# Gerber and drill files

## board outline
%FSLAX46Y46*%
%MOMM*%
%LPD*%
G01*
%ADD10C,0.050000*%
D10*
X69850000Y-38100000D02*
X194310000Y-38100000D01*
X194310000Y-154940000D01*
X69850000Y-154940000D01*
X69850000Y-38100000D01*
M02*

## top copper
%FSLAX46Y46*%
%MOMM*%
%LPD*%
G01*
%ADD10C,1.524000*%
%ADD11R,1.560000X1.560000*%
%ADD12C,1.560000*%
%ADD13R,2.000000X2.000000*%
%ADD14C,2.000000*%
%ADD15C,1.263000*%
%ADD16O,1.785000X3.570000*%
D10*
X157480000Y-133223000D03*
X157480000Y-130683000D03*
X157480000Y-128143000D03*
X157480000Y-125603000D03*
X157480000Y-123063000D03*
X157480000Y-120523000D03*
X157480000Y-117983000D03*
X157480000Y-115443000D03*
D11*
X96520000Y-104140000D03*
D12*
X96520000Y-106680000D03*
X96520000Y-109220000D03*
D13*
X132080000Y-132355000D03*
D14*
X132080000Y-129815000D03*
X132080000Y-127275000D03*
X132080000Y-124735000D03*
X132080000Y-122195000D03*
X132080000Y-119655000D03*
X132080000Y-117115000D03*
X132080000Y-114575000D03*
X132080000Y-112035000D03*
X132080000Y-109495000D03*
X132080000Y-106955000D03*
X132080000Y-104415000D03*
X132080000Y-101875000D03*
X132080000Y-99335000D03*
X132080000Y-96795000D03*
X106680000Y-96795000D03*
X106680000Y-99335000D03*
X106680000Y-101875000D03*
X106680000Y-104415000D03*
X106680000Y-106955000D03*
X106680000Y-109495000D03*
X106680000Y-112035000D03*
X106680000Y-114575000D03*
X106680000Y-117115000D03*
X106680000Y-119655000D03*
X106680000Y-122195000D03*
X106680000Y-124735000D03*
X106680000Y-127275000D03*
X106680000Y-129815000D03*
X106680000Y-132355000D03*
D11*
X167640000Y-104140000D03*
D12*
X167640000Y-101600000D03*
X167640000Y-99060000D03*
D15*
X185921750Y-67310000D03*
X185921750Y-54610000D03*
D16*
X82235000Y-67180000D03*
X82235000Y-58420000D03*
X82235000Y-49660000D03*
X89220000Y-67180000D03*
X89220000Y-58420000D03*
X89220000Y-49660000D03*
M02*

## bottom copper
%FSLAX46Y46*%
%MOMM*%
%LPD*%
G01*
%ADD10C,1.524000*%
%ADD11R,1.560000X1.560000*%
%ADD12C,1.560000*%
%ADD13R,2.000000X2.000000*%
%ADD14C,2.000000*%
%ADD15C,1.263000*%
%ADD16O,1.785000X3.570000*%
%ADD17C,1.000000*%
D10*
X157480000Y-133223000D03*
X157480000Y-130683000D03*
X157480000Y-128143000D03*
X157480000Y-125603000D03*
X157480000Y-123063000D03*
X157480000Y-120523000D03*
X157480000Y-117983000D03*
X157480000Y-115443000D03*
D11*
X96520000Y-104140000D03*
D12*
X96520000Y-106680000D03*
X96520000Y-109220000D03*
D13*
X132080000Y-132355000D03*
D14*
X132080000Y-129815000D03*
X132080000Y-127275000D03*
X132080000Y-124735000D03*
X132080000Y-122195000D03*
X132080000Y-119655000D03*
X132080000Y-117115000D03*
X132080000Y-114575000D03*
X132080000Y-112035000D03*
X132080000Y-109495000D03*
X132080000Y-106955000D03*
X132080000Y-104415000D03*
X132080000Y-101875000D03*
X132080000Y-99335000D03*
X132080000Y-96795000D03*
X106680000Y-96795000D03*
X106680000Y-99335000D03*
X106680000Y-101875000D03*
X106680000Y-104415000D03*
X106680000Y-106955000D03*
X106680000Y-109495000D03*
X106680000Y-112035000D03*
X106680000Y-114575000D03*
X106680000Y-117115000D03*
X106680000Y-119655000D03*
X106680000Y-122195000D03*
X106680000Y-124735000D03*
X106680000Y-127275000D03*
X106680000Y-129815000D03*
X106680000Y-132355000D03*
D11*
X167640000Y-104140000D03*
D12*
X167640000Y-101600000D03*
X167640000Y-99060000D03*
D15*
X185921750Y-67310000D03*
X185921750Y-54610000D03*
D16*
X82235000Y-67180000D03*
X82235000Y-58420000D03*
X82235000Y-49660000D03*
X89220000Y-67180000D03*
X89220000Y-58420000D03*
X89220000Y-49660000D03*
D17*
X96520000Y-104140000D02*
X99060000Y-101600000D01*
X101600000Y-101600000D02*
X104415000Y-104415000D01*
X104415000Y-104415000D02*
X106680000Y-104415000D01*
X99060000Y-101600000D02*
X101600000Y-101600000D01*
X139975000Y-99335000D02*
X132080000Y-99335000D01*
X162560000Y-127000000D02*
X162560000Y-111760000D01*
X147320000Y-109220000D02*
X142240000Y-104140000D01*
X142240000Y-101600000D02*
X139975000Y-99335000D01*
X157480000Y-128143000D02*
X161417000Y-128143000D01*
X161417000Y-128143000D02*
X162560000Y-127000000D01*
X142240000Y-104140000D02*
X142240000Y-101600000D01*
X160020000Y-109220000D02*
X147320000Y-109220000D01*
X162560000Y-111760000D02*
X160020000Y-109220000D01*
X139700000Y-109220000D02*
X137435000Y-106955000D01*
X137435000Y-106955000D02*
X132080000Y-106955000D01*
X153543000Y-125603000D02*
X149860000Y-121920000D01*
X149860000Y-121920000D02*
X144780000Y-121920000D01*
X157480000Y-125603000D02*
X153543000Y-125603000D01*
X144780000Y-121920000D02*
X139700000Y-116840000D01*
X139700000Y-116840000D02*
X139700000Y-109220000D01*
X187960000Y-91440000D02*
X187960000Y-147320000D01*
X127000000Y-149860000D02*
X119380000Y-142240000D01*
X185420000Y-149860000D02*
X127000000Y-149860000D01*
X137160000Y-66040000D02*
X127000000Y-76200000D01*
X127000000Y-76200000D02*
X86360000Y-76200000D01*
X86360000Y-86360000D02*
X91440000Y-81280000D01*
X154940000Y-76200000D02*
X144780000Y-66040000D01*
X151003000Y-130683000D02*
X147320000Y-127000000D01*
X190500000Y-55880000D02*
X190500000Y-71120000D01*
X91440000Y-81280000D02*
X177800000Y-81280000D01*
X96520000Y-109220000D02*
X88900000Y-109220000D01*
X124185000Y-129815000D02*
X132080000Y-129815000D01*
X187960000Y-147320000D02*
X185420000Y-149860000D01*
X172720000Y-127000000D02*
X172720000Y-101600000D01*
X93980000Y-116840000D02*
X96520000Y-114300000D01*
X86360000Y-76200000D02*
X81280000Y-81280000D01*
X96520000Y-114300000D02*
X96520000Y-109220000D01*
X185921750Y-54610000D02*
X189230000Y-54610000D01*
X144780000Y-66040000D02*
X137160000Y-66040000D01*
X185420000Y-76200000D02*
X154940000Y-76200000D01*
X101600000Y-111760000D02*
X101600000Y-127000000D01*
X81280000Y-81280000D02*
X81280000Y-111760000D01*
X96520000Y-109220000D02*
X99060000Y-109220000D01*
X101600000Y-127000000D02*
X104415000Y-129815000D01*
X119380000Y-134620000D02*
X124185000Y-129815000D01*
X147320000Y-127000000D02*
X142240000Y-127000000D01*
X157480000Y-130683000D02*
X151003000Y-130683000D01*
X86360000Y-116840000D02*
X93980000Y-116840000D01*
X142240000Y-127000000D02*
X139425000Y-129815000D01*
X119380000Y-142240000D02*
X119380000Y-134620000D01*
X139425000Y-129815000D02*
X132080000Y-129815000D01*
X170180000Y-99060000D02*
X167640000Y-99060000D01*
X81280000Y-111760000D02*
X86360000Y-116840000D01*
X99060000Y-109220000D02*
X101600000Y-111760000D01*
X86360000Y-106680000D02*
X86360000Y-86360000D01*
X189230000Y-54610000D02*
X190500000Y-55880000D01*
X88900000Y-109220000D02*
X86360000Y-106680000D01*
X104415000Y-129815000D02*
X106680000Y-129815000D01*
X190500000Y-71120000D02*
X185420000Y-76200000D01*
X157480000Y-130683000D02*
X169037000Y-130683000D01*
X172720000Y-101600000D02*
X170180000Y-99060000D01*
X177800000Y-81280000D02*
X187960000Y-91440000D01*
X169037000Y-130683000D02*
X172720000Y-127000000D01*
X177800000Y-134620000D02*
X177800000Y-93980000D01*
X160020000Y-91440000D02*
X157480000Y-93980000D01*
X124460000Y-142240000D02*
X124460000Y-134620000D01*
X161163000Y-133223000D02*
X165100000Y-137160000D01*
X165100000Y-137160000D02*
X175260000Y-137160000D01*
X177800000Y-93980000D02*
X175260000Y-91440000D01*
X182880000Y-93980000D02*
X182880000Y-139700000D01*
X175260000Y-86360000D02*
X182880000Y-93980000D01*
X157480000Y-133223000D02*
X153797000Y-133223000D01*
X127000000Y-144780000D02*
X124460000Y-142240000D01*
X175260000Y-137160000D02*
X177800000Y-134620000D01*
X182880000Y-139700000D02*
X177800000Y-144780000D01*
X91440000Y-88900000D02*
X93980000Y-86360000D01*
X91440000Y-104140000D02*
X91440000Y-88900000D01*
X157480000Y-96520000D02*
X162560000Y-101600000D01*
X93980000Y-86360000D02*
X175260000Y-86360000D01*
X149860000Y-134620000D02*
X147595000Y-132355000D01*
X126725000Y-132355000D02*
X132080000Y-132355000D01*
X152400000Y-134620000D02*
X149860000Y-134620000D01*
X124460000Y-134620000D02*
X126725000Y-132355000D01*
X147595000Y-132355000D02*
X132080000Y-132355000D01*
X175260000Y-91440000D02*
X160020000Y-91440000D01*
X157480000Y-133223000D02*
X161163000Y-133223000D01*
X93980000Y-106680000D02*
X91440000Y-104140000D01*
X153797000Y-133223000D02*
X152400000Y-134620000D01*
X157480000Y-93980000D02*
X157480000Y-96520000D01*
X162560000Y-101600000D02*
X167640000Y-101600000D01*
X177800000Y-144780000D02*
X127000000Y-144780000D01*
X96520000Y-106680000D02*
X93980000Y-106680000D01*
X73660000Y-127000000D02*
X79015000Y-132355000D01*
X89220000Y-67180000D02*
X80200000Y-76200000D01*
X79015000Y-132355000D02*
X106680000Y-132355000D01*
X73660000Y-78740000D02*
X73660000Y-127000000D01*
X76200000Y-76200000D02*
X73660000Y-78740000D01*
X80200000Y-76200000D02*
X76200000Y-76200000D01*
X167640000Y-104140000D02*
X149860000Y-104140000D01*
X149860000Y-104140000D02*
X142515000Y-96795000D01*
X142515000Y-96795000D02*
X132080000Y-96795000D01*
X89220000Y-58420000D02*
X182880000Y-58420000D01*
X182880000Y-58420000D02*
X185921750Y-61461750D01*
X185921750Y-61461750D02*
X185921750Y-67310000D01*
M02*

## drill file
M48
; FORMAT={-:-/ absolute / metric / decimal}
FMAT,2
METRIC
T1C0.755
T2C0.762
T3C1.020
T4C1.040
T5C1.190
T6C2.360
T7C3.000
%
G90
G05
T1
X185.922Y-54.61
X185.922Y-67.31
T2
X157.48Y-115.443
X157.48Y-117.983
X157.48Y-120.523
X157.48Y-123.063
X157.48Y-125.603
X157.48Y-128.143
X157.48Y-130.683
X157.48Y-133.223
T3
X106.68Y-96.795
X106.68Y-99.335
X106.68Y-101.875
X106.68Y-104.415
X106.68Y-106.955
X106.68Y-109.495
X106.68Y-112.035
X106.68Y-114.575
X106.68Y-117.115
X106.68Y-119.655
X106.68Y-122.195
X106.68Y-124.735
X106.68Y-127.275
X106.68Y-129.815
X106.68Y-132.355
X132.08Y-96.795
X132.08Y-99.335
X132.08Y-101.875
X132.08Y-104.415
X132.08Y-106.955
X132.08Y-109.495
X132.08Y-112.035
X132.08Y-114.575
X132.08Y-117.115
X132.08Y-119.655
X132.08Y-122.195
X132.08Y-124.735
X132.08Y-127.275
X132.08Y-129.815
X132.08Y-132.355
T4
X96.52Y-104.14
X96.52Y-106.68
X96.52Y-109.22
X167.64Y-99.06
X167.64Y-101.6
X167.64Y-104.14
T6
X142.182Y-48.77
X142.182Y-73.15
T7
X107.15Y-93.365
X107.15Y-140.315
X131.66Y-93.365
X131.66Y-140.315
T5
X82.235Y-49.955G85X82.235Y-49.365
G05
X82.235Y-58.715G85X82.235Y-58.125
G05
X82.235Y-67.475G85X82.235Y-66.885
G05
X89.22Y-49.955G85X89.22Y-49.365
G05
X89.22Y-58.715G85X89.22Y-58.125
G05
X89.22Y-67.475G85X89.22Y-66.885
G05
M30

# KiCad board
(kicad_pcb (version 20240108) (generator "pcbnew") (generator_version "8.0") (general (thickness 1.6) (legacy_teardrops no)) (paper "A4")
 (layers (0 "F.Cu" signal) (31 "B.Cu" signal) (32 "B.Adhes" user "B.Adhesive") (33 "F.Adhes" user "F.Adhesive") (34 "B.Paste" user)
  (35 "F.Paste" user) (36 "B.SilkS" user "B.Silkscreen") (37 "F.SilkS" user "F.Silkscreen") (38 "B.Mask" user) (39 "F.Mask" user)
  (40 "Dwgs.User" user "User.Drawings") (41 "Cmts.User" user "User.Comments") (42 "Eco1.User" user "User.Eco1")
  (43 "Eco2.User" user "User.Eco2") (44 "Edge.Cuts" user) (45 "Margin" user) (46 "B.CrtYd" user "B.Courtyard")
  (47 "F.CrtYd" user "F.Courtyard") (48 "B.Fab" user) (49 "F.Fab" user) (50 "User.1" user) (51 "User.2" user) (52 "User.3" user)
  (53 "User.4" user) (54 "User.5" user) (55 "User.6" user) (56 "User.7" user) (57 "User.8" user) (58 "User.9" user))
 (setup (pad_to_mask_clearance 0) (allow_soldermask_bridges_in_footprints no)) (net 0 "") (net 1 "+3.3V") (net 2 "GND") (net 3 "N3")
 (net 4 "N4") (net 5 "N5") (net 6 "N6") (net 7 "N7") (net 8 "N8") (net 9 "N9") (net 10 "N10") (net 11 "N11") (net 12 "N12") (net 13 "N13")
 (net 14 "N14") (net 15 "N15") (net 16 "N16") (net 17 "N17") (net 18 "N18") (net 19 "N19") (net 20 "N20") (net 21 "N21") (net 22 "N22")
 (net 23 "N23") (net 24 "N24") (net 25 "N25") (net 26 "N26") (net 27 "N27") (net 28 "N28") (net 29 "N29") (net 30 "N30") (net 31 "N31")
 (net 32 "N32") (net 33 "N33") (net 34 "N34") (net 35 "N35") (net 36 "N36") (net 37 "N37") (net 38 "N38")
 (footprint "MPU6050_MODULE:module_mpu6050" (layer "F.Cu") (at 157.48 115.443 180)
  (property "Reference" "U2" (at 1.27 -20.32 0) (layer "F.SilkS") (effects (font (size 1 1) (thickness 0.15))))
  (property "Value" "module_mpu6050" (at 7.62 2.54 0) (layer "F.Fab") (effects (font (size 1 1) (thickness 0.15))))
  (pad "1" thru_hole circle (at 0 -17.78 180) (size 1.524 1.524) (drill 0.762) (layers "*.Cu" "*.Mask") (remove_unused_layers no)
   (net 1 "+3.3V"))
  (pad "2" thru_hole circle (at 0 -15.24 180) (size 1.524 1.524) (drill 0.762) (layers "*.Cu" "*.Mask") (remove_unused_layers no)
   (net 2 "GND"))
  (pad "3" thru_hole circle (at 0 -12.7 180) (size 1.524 1.524) (drill 0.762) (layers "*.Cu" "*.Mask") (remove_unused_layers no)
   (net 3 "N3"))
  (pad "4" thru_hole circle (at 0 -10.16 180) (size 1.524 1.524) (drill 0.762) (layers "*.Cu" "*.Mask") (remove_unused_layers no)
   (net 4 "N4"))
  (pad "5" thru_hole circle (at 0 -7.62 180) (size 1.524 1.524) (drill 0.762) (layers "*.Cu" "*.Mask") (remove_unused_layers no)
   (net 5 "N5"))
  (pad "6" thru_hole circle (at 0 -5.08 180) (size 1.524 1.524) (drill 0.762) (layers "*.Cu" "*.Mask") (remove_unused_layers no)
   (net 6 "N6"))
  (pad "7" thru_hole circle (at 0 -2.54 180) (size 1.524 1.524) (drill 0.762) (layers "*.Cu" "*.Mask") (remove_unused_layers no)
   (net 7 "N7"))
  (pad "8" thru_hole circle (at 0 0 180) (size 1.524 1.524) (drill 0.762) (layers "*.Cu" "*.Mask") (remove_unused_layers no) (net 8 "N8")))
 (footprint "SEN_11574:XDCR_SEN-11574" (layer "F.Cu") (at 96.52 106.68 180)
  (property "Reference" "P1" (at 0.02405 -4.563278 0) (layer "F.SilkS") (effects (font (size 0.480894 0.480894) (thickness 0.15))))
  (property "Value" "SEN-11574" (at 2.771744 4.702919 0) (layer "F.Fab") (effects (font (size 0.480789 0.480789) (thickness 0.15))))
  (pad "1" thru_hole rect (at 0 2.54 180) (size 1.56 1.56) (drill 1.04) (layers "*.Cu" "*.Mask") (remove_unused_layers no) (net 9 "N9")
   (solder_mask_margin 0.102))
  (pad "2" thru_hole circle (at 0 0 180) (size 1.56 1.56) (drill 1.04) (layers "*.Cu" "*.Mask") (remove_unused_layers no) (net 1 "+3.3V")
   (solder_mask_margin 0.102))
  (pad "3" thru_hole circle (at 0 -2.54 180) (size 1.56 1.56) (drill 1.04) (layers "*.Cu" "*.Mask") (remove_unused_layers no) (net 2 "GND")
   (solder_mask_margin 0.102)))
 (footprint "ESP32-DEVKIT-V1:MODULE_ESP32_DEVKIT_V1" (layer "F.Cu") (at 119.38 116.84 180)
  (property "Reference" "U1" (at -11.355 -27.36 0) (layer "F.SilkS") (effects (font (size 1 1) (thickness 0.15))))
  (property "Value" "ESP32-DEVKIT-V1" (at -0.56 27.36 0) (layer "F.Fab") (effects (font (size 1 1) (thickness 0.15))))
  (pad "" np_thru_hole circle (at -12.28 -23.475 180) (size 3 3) (drill 3) (layers "*.Cu" "*.Mask"))
  (pad "" np_thru_hole circle (at -12.28 23.475 180) (size 3 3) (drill 3) (layers "*.Cu" "*.Mask"))
  (pad "" np_thru_hole circle (at 12.23 -23.475 180) (size 3 3) (drill 3) (layers "*.Cu" "*.Mask"))
  (pad "" np_thru_hole circle (at 12.23 23.475 180) (size 3 3) (drill 3) (layers "*.Cu" "*.Mask"))
  (pad "1" thru_hole rect (at -12.7 -15.515 180) (size 2 2) (drill 1.02) (layers "*.Cu" "*.Mask") (remove_unused_layers no) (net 1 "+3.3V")
   (solder_mask_margin 0.102))
  (pad "2" thru_hole circle (at -12.7 -12.975 180) (size 2 2) (drill 1.02) (layers "*.Cu" "*.Mask") (remove_unused_layers no) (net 2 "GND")
   (solder_mask_margin 0.102))
  (pad "3" thru_hole circle (at -12.7 -10.435 180) (size 2 2) (drill 1.02) (layers "*.Cu" "*.Mask") (remove_unused_layers no) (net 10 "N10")
   (solder_mask_margin 0.102))
  (pad "4" thru_hole circle (at -12.7 -7.895 180) (size 2 2) (drill 1.02) (layers "*.Cu" "*.Mask") (remove_unused_layers no) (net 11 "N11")
   (solder_mask_margin 0.102))
  (pad "5" thru_hole circle (at -12.7 -5.355 180) (size 2 2) (drill 1.02) (layers "*.Cu" "*.Mask") (remove_unused_layers no) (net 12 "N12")
   (solder_mask_margin 0.102))
  (pad "6" thru_hole circle (at -12.7 -2.815 180) (size 2 2) (drill 1.02) (layers "*.Cu" "*.Mask") (remove_unused_layers no) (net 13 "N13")
   (solder_mask_margin 0.102))
  (pad "7" thru_hole circle (at -12.7 -0.275 180) (size 2 2) (drill 1.02) (layers "*.Cu" "*.Mask") (remove_unused_layers no) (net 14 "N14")
   (solder_mask_margin 0.102))
  (pad "8" thru_hole circle (at -12.7 2.265 180) (size 2 2) (drill 1.02) (layers "*.Cu" "*.Mask") (remove_unused_layers no) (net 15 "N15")
   (solder_mask_margin 0.102))
  (pad "9" thru_hole circle (at -12.7 4.805 180) (size 2 2) (drill 1.02) (layers "*.Cu" "*.Mask") (remove_unused_layers no) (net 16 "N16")
   (solder_mask_margin 0.102))
  (pad "10" thru_hole circle (at -12.7 7.345 180) (size 2 2) (drill 1.02) (layers "*.Cu" "*.Mask") (remove_unused_layers no) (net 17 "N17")
   (solder_mask_margin 0.102))
  (pad "11" thru_hole circle (at -12.7 9.885 180) (size 2 2) (drill 1.02) (layers "*.Cu" "*.Mask") (remove_unused_layers no) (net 4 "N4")
   (solder_mask_margin 0.102))
  (pad "12" thru_hole circle (at -12.7 12.425 180) (size 2 2) (drill 1.02) (layers "*.Cu" "*.Mask") (remove_unused_layers no) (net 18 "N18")
   (solder_mask_margin 0.102))
  (pad "13" thru_hole circle (at -12.7 14.965 180) (size 2 2) (drill 1.02) (layers "*.Cu" "*.Mask") (remove_unused_layers no) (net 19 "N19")
   (solder_mask_margin 0.102))
  (pad "14" thru_hole circle (at -12.7 17.505 180) (size 2 2) (drill 1.02) (layers "*.Cu" "*.Mask") (remove_unused_layers no) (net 3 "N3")
   (solder_mask_margin 0.102))
  (pad "15" thru_hole circle (at -12.7 20.045 180) (size 2 2) (drill 1.02) (layers "*.Cu" "*.Mask") (remove_unused_layers no) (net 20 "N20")
   (solder_mask_margin 0.102))
  (pad "16" thru_hole circle (at 12.7 20.045 180) (size 2 2) (drill 1.02) (layers "*.Cu" "*.Mask") (remove_unused_layers no) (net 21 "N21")
   (solder_mask_margin 0.102))
  (pad "17" thru_hole circle (at 12.7 17.505 180) (size 2 2) (drill 1.02) (layers "*.Cu" "*.Mask") (remove_unused_layers no) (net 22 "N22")
   (solder_mask_margin 0.102))
  (pad "18" thru_hole circle (at 12.7 14.965 180) (size 2 2) (drill 1.02) (layers "*.Cu" "*.Mask") (remove_unused_layers no) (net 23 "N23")
   (solder_mask_margin 0.102))
  (pad "19" thru_hole circle (at 12.7 12.425 180) (size 2 2) (drill 1.02) (layers "*.Cu" "*.Mask") (remove_unused_layers no) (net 9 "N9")
   (solder_mask_margin 0.102))
  (pad "20" thru_hole circle (at 12.7 9.885 180) (size 2 2) (drill 1.02) (layers "*.Cu" "*.Mask") (remove_unused_layers no) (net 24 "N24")
   (solder_mask_margin 0.102))
  (pad "21" thru_hole circle (at 12.7 7.345 180) (size 2 2) (drill 1.02) (layers "*.Cu" "*.Mask") (remove_unused_layers no) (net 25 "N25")
   (solder_mask_margin 0.102))
  (pad "22" thru_hole circle (at 12.7 4.805 180) (size 2 2) (drill 1.02) (layers "*.Cu" "*.Mask") (remove_unused_layers no) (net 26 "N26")
   (solder_mask_margin 0.102))
  (pad "23" thru_hole circle (at 12.7 2.265 180) (size 2 2) (drill 1.02) (layers "*.Cu" "*.Mask") (remove_unused_layers no) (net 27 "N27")
   (solder_mask_margin 0.102))
  (pad "24" thru_hole circle (at 12.7 -0.275 180) (size 2 2) (drill 1.02) (layers "*.Cu" "*.Mask") (remove_unused_layers no) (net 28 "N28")
   (solder_mask_margin 0.102))
  (pad "25" thru_hole circle (at 12.7 -2.815 180) (size 2 2) (drill 1.02) (layers "*.Cu" "*.Mask") (remove_unused_layers no) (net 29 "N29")
   (solder_mask_margin 0.102))
  (pad "26" thru_hole circle (at 12.7 -5.355 180) (size 2 2) (drill 1.02) (layers "*.Cu" "*.Mask") (remove_unused_layers no) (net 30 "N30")
   (solder_mask_margin 0.102))
  (pad "27" thru_hole circle (at 12.7 -7.895 180) (size 2 2) (drill 1.02) (layers "*.Cu" "*.Mask") (remove_unused_layers no) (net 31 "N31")
   (solder_mask_margin 0.102))
  (pad "28" thru_hole circle (at 12.7 -10.435 180) (size 2 2) (drill 1.02) (layers "*.Cu" "*.Mask") (remove_unused_layers no) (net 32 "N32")
   (solder_mask_margin 0.102))
  (pad "29" thru_hole circle (at 12.7 -12.975 180) (size 2 2) (drill 1.02) (layers "*.Cu" "*.Mask") (remove_unused_layers no) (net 2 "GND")
   (solder_mask_margin 0.102))
  (pad "30" thru_hole circle (at 12.7 -15.515 180) (size 2 2) (drill 1.02) (layers "*.Cu" "*.Mask") (remove_unused_layers no) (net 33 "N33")
   (solder_mask_margin 0.102))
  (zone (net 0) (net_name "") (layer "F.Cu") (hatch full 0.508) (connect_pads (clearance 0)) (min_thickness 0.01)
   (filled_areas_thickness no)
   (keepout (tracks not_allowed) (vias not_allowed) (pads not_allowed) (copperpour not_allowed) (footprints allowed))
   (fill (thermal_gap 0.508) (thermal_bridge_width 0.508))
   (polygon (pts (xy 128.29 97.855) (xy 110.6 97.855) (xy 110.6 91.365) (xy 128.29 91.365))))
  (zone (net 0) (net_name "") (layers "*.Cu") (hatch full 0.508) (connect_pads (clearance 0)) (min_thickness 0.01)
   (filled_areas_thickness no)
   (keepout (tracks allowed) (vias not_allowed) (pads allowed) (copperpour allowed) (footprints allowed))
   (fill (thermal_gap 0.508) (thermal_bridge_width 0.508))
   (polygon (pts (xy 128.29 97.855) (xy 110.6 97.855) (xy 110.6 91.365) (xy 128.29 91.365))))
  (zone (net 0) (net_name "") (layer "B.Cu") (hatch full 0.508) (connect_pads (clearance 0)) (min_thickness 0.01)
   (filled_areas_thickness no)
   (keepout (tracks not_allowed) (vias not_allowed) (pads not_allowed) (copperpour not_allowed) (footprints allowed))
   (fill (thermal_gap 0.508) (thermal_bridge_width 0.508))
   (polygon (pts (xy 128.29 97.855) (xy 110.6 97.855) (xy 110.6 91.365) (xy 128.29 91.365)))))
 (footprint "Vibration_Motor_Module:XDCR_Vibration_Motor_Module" (layer "F.Cu") (at 175.26 101.6)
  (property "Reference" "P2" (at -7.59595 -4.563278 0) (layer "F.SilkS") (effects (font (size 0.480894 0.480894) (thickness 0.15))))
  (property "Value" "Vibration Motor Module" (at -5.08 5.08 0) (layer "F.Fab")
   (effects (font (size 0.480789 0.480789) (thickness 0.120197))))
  (pad "1" thru_hole rect (at -7.62 2.54) (size 1.56 1.56) (drill 1.04) (layers "*.Cu" "*.Mask") (remove_unused_layers no) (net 20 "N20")
   (solder_mask_margin 0.102))
  (pad "2" thru_hole circle (at -7.62 0) (size 1.56 1.56) (drill 1.04) (layers "*.Cu" "*.Mask") (remove_unused_layers no) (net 1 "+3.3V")
   (solder_mask_margin 0.102))
  (pad "3" thru_hole circle (at -7.62 -2.54) (size 1.56 1.56) (drill 1.04) (layers "*.Cu" "*.Mask") (remove_unused_layers no) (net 2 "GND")
   (solder_mask_margin 0.102)))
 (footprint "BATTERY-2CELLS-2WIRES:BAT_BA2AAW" (layer "F.Cu") (at 142.18175 60.96)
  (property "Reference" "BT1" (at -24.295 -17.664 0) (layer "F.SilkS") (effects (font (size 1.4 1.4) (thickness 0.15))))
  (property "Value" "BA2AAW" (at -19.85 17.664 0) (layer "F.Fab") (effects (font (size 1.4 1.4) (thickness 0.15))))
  (pad "" np_thru_hole circle (at 0 -12.19) (size 2.36 2.36) (drill 2.36) (layers "*.Cu" "*.Mask"))
  (pad "" np_thru_hole circle (at 0 12.19) (size 2.36 2.36) (drill 2.36) (layers "*.Cu" "*.Mask"))
  (pad "+" thru_hole circle (at 43.74 6.35) (size 1.263 1.263) (drill 0.755) (layers "*.Cu" "*.Mask") (remove_unused_layers no)
   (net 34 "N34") (solder_mask_margin 0.102))
  (pad "-" thru_hole circle (at 43.74 -6.35) (size 1.263 1.263) (drill 0.755) (layers "*.Cu" "*.Mask") (remove_unused_layers no)
   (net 2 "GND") (solder_mask_margin 0.102)))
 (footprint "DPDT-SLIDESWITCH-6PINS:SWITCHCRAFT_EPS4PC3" (layer "F.Cu") (at 101.6 58.42 90)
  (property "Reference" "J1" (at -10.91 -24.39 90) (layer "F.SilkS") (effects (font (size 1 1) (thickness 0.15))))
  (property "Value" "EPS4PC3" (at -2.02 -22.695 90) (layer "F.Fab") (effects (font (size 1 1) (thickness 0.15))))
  (pad "1" thru_hole oval (at -8.76 -19.365 90) (size 3.57 1.785) (drill oval 1.78 1.19) (layers "*.Cu" "*.Mask") (remove_unused_layers no)
   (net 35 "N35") (solder_mask_margin 0.102))
  (pad "2" thru_hole oval (at 0 -19.365 90) (size 3.57 1.785) (drill oval 1.78 1.19) (layers "*.Cu" "*.Mask") (remove_unused_layers no)
   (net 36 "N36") (solder_mask_margin 0.102))
  (pad "3" thru_hole oval (at 8.76 -19.365 90) (size 3.57 1.785) (drill oval 1.78 1.19) (layers "*.Cu" "*.Mask") (remove_unused_layers no)
   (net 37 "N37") (solder_mask_margin 0.102))
  (pad "4" thru_hole oval (at -8.76 -12.38 90) (size 3.57 1.785) (drill oval 1.78 1.19) (layers "*.Cu" "*.Mask") (remove_unused_layers no)
   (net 33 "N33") (solder_mask_margin 0.102))
  (pad "5" thru_hole oval (at 0 -12.38 90) (size 3.57 1.785) (drill oval 1.78 1.19) (layers "*.Cu" "*.Mask") (remove_unused_layers no)
   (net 34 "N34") (solder_mask_margin 0.102))
  (pad "6" thru_hole oval (at 8.76 -12.38 90) (size 3.57 1.785) (drill oval 1.78 1.19) (layers "*.Cu" "*.Mask") (remove_unused_layers no)
   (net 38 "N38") (solder_mask_margin 0.102)))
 (gr_rect (start 69.85 38.1) (end 194.31 154.94) (stroke (width 0.05) (type default)) (fill none) (layer "Edge.Cuts"))
 (segment (start 96.52 104.14) (end 99.06 101.6) (width 1) (layer "B.Cu") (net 9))
 (segment (start 101.6 101.6) (end 104.415 104.415) (width 1) (layer "B.Cu") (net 9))
 (segment (start 104.415 104.415) (end 106.68 104.415) (width 1) (layer "B.Cu") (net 9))
 (segment (start 99.06 101.6) (end 101.6 101.6) (width 1) (layer "B.Cu") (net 9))
 (segment (start 139.975 99.335) (end 132.08 99.335) (width 1) (layer "B.Cu") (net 3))
 (segment (start 162.56 127) (end 162.56 111.76) (width 1) (layer "B.Cu") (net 3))
 (segment (start 147.32 109.22) (end 142.24 104.14) (width 1) (layer "B.Cu") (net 3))
 (segment (start 142.24 101.6) (end 139.975 99.335) (width 1) (layer "B.Cu") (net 3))
 (segment (start 157.48 128.143) (end 161.417 128.143) (width 1) (layer "B.Cu") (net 3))
 (segment (start 161.417 128.143) (end 162.56 127) (width 1) (layer "B.Cu") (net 3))
 (segment (start 142.24 104.14) (end 142.24 101.6) (width 1) (layer "B.Cu") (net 3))
 (segment (start 160.02 109.22) (end 147.32 109.22) (width 1) (layer "B.Cu") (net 3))
 (segment (start 162.56 111.76) (end 160.02 109.22) (width 1) (layer "B.Cu") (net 3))
 (segment (start 139.7 109.22) (end 137.435 106.955) (width 1) (layer "B.Cu") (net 4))
 (segment (start 137.435 106.955) (end 132.08 106.955) (width 1) (layer "B.Cu") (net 4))
 (segment (start 153.543 125.603) (end 149.86 121.92) (width 1) (layer "B.Cu") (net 4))
 (segment (start 149.86 121.92) (end 144.78 121.92) (width 1) (layer "B.Cu") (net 4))
 (segment (start 157.48 125.603) (end 153.543 125.603) (width 1) (layer "B.Cu") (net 4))
 (segment (start 144.78 121.92) (end 139.7 116.84) (width 1) (layer "B.Cu") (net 4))
 (segment (start 139.7 116.84) (end 139.7 109.22) (width 1) (layer "B.Cu") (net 4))
 (segment (start 187.96 91.44) (end 187.96 147.32) (width 1) (layer "B.Cu") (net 2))
 (segment (start 127 149.86) (end 119.38 142.24) (width 1) (layer "B.Cu") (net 2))
 (segment (start 185.42 149.86) (end 127 149.86) (width 1) (layer "B.Cu") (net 2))
 (segment (start 137.16 66.04) (end 127 76.2) (width 1) (layer "B.Cu") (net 2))
 (segment (start 127 76.2) (end 86.36 76.2) (width 1) (layer "B.Cu") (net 2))
 (segment (start 86.36 86.36) (end 91.44 81.28) (width 1) (layer "B.Cu") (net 2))
 (segment (start 154.94 76.2) (end 144.78 66.04) (width 1) (layer "B.Cu") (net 2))
 (segment (start 151.003 130.683) (end 147.32 127) (width 1) (layer "B.Cu") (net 2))
 (segment (start 190.5 55.88) (end 190.5 71.12) (width 1) (layer "B.Cu") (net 2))
 (segment (start 91.44 81.28) (end 177.8 81.28) (width 1) (layer "B.Cu") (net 2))
 (segment (start 96.52 109.22) (end 88.9 109.22) (width 1) (layer "B.Cu") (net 2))
 (segment (start 124.185 129.815) (end 132.08 129.815) (width 1) (layer "B.Cu") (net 2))
 (segment (start 187.96 147.32) (end 185.42 149.86) (width 1) (layer "B.Cu") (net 2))
 (segment (start 172.72 127) (end 172.72 101.6) (width 1) (layer "B.Cu") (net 2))
 (segment (start 93.98 116.84) (end 96.52 114.3) (width 1) (layer "B.Cu") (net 2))
 (segment (start 86.36 76.2) (end 81.28 81.28) (width 1) (layer "B.Cu") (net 2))
 (segment (start 96.52 114.3) (end 96.52 109.22) (width 1) (layer "B.Cu") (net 2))
 (segment (start 185.92175 54.61) (end 189.23 54.61) (width 1) (layer "B.Cu") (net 2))
 (segment (start 144.78 66.04) (end 137.16 66.04) (width 1) (layer "B.Cu") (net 2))
 (segment (start 185.42 76.2) (end 154.94 76.2) (width 1) (layer "B.Cu") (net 2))
 (segment (start 101.6 111.76) (end 101.6 127) (width 1) (layer "B.Cu") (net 2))
 (segment (start 81.28 81.28) (end 81.28 111.76) (width 1) (layer "B.Cu") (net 2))
 (segment (start 96.52 109.22) (end 99.06 109.22) (width 1) (layer "B.Cu") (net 2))
 (segment (start 101.6 127) (end 104.415 129.815) (width 1) (layer "B.Cu") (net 2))
 (segment (start 119.38 134.62) (end 124.185 129.815) (width 1) (layer "B.Cu") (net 2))
 (segment (start 147.32 127) (end 142.24 127) (width 1) (layer "B.Cu") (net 2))
 (segment (start 157.48 130.683) (end 151.003 130.683) (width 1) (layer "B.Cu") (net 2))
 (segment (start 86.36 116.84) (end 93.98 116.84) (width 1) (layer "B.Cu") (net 2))
 (segment (start 142.24 127) (end 139.425 129.815) (width 1) (layer "B.Cu") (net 2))
 (segment (start 119.38 142.24) (end 119.38 134.62) (width 1) (layer "B.Cu") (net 2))
 (segment (start 139.425 129.815) (end 132.08 129.815) (width 1) (layer "B.Cu") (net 2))
 (segment (start 170.18 99.06) (end 167.64 99.06) (width 1) (layer "B.Cu") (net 2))
 (segment (start 81.28 111.76) (end 86.36 116.84) (width 1) (layer "B.Cu") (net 2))
 (segment (start 99.06 109.22) (end 101.6 111.76) (width 1) (layer "B.Cu") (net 2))
 (segment (start 86.36 106.68) (end 86.36 86.36) (width 1) (layer "B.Cu") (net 2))
 (segment (start 189.23 54.61) (end 190.5 55.88) (width 1) (layer "B.Cu") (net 2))
 (segment (start 88.9 109.22) (end 86.36 106.68) (width 1) (layer "B.Cu") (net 2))
 (segment (start 104.415 129.815) (end 106.68 129.815) (width 1) (layer "B.Cu") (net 2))
 (segment (start 190.5 71.12) (end 185.42 76.2) (width 1) (layer "B.Cu") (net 2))
 (segment (start 157.48 130.683) (end 169.037 130.683) (width 1) (layer "B.Cu") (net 2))
 (segment (start 172.72 101.6) (end 170.18 99.06) (width 1) (layer "B.Cu") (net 2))
 (segment (start 177.8 81.28) (end 187.96 91.44) (width 1) (layer "B.Cu") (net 2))
 (segment (start 169.037 130.683) (end 172.72 127) (width 1) (layer "B.Cu") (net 2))
 (segment (start 177.8 134.62) (end 177.8 93.98) (width 1) (layer "B.Cu") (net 1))
 (segment (start 160.02 91.44) (end 157.48 93.98) (width 1) (layer "B.Cu") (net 1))
 (segment (start 124.46 142.24) (end 124.46 134.62) (width 1) (layer "B.Cu") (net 1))
 (segment (start 161.163 133.223) (end 165.1 137.16) (width 1) (layer "B.Cu") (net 1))
 (segment (start 165.1 137.16) (end 175.26 137.16) (width 1) (layer "B.Cu") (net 1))
 (segment (start 177.8 93.98) (end 175.26 91.44) (width 1) (layer "B.Cu") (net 1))
 (segment (start 182.88 93.98) (end 182.88 139.7) (width 1) (layer "B.Cu") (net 1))
 (segment (start 175.26 86.36) (end 182.88 93.98) (width 1) (layer "B.Cu") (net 1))
 (segment (start 157.48 133.223) (end 153.797 133.223) (width 1) (layer "B.Cu") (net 1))
 (segment (start 127 144.78) (end 124.46 142.24) (width 1) (layer "B.Cu") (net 1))
 (segment (start 175.26 137.16) (end 177.8 134.62) (width 1) (layer "B.Cu") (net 1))
 (segment (start 182.88 139.7) (end 177.8 144.78) (width 1) (layer "B.Cu") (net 1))
 (segment (start 91.44 88.9) (end 93.98 86.36) (width 1) (layer "B.Cu") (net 1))
 (segment (start 91.44 104.14) (end 91.44 88.9) (width 1) (layer "B.Cu") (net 1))
 (segment (start 157.48 96.52) (end 162.56 101.6) (width 1) (layer "B.Cu") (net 1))
 (segment (start 93.98 86.36) (end 175.26 86.36) (width 1) (layer "B.Cu") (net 1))
 (segment (start 149.86 134.62) (end 147.595 132.355) (width 1) (layer "B.Cu") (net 1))
 (segment (start 126.725 132.355) (end 132.08 132.355) (width 1) (layer "B.Cu") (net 1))
 (segment (start 152.4 134.62) (end 149.86 134.62) (width 1) (layer "B.Cu") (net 1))
 (segment (start 124.46 134.62) (end 126.725 132.355) (width 1) (layer "B.Cu") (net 1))
 (segment (start 147.595 132.355) (end 132.08 132.355) (width 1) (layer "B.Cu") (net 1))
 (segment (start 175.26 91.44) (end 160.02 91.44) (width 1) (layer "B.Cu") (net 1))
 (segment (start 157.48 133.223) (end 161.163 133.223) (width 1) (layer "B.Cu") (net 1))
 (segment (start 93.98 106.68) (end 91.44 104.14) (width 1) (layer "B.Cu") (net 1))
 (segment (start 153.797 133.223) (end 152.4 134.62) (width 1) (layer "B.Cu") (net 1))
 (segment (start 157.48 93.98) (end 157.48 96.52) (width 1) (layer "B.Cu") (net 1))
 (segment (start 162.56 101.6) (end 167.64 101.6) (width 1) (layer "B.Cu") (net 1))
 (segment (start 177.8 144.78) (end 127 144.78) (width 1) (layer "B.Cu") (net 1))
 (segment (start 96.52 106.68) (end 93.98 106.68) (width 1) (layer "B.Cu") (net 1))
 (segment (start 73.66 127) (end 79.015 132.355) (width 1) (layer "B.Cu") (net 33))
 (segment (start 89.22 67.18) (end 80.2 76.2) (width 1) (layer "B.Cu") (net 33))
 (segment (start 79.015 132.355) (end 106.68 132.355) (width 1) (layer "B.Cu") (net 33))
 (segment (start 73.66 78.74) (end 73.66 127) (width 1) (layer "B.Cu") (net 33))
 (segment (start 76.2 76.2) (end 73.66 78.74) (width 1) (layer "B.Cu") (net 33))
 (segment (start 80.2 76.2) (end 76.2 76.2) (width 1) (layer "B.Cu") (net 33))
 (segment (start 167.64 104.14) (end 149.86 104.14) (width 1) (layer "B.Cu") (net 20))
 (segment (start 149.86 104.14) (end 142.515 96.795) (width 1) (layer "B.Cu") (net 20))
 (segment (start 142.515 96.795) (end 132.08 96.795) (width 1) (layer "B.Cu") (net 20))
 (segment (start 89.22 58.42) (end 182.88 58.42) (width 1) (layer "B.Cu") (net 34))
 (segment (start 182.88 58.42) (end 185.92175 61.46175) (width 1) (layer "B.Cu") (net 34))
 (segment (start 185.92175 61.46175) (end 185.92175 67.31) (width 1) (layer "B.Cu") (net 34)))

